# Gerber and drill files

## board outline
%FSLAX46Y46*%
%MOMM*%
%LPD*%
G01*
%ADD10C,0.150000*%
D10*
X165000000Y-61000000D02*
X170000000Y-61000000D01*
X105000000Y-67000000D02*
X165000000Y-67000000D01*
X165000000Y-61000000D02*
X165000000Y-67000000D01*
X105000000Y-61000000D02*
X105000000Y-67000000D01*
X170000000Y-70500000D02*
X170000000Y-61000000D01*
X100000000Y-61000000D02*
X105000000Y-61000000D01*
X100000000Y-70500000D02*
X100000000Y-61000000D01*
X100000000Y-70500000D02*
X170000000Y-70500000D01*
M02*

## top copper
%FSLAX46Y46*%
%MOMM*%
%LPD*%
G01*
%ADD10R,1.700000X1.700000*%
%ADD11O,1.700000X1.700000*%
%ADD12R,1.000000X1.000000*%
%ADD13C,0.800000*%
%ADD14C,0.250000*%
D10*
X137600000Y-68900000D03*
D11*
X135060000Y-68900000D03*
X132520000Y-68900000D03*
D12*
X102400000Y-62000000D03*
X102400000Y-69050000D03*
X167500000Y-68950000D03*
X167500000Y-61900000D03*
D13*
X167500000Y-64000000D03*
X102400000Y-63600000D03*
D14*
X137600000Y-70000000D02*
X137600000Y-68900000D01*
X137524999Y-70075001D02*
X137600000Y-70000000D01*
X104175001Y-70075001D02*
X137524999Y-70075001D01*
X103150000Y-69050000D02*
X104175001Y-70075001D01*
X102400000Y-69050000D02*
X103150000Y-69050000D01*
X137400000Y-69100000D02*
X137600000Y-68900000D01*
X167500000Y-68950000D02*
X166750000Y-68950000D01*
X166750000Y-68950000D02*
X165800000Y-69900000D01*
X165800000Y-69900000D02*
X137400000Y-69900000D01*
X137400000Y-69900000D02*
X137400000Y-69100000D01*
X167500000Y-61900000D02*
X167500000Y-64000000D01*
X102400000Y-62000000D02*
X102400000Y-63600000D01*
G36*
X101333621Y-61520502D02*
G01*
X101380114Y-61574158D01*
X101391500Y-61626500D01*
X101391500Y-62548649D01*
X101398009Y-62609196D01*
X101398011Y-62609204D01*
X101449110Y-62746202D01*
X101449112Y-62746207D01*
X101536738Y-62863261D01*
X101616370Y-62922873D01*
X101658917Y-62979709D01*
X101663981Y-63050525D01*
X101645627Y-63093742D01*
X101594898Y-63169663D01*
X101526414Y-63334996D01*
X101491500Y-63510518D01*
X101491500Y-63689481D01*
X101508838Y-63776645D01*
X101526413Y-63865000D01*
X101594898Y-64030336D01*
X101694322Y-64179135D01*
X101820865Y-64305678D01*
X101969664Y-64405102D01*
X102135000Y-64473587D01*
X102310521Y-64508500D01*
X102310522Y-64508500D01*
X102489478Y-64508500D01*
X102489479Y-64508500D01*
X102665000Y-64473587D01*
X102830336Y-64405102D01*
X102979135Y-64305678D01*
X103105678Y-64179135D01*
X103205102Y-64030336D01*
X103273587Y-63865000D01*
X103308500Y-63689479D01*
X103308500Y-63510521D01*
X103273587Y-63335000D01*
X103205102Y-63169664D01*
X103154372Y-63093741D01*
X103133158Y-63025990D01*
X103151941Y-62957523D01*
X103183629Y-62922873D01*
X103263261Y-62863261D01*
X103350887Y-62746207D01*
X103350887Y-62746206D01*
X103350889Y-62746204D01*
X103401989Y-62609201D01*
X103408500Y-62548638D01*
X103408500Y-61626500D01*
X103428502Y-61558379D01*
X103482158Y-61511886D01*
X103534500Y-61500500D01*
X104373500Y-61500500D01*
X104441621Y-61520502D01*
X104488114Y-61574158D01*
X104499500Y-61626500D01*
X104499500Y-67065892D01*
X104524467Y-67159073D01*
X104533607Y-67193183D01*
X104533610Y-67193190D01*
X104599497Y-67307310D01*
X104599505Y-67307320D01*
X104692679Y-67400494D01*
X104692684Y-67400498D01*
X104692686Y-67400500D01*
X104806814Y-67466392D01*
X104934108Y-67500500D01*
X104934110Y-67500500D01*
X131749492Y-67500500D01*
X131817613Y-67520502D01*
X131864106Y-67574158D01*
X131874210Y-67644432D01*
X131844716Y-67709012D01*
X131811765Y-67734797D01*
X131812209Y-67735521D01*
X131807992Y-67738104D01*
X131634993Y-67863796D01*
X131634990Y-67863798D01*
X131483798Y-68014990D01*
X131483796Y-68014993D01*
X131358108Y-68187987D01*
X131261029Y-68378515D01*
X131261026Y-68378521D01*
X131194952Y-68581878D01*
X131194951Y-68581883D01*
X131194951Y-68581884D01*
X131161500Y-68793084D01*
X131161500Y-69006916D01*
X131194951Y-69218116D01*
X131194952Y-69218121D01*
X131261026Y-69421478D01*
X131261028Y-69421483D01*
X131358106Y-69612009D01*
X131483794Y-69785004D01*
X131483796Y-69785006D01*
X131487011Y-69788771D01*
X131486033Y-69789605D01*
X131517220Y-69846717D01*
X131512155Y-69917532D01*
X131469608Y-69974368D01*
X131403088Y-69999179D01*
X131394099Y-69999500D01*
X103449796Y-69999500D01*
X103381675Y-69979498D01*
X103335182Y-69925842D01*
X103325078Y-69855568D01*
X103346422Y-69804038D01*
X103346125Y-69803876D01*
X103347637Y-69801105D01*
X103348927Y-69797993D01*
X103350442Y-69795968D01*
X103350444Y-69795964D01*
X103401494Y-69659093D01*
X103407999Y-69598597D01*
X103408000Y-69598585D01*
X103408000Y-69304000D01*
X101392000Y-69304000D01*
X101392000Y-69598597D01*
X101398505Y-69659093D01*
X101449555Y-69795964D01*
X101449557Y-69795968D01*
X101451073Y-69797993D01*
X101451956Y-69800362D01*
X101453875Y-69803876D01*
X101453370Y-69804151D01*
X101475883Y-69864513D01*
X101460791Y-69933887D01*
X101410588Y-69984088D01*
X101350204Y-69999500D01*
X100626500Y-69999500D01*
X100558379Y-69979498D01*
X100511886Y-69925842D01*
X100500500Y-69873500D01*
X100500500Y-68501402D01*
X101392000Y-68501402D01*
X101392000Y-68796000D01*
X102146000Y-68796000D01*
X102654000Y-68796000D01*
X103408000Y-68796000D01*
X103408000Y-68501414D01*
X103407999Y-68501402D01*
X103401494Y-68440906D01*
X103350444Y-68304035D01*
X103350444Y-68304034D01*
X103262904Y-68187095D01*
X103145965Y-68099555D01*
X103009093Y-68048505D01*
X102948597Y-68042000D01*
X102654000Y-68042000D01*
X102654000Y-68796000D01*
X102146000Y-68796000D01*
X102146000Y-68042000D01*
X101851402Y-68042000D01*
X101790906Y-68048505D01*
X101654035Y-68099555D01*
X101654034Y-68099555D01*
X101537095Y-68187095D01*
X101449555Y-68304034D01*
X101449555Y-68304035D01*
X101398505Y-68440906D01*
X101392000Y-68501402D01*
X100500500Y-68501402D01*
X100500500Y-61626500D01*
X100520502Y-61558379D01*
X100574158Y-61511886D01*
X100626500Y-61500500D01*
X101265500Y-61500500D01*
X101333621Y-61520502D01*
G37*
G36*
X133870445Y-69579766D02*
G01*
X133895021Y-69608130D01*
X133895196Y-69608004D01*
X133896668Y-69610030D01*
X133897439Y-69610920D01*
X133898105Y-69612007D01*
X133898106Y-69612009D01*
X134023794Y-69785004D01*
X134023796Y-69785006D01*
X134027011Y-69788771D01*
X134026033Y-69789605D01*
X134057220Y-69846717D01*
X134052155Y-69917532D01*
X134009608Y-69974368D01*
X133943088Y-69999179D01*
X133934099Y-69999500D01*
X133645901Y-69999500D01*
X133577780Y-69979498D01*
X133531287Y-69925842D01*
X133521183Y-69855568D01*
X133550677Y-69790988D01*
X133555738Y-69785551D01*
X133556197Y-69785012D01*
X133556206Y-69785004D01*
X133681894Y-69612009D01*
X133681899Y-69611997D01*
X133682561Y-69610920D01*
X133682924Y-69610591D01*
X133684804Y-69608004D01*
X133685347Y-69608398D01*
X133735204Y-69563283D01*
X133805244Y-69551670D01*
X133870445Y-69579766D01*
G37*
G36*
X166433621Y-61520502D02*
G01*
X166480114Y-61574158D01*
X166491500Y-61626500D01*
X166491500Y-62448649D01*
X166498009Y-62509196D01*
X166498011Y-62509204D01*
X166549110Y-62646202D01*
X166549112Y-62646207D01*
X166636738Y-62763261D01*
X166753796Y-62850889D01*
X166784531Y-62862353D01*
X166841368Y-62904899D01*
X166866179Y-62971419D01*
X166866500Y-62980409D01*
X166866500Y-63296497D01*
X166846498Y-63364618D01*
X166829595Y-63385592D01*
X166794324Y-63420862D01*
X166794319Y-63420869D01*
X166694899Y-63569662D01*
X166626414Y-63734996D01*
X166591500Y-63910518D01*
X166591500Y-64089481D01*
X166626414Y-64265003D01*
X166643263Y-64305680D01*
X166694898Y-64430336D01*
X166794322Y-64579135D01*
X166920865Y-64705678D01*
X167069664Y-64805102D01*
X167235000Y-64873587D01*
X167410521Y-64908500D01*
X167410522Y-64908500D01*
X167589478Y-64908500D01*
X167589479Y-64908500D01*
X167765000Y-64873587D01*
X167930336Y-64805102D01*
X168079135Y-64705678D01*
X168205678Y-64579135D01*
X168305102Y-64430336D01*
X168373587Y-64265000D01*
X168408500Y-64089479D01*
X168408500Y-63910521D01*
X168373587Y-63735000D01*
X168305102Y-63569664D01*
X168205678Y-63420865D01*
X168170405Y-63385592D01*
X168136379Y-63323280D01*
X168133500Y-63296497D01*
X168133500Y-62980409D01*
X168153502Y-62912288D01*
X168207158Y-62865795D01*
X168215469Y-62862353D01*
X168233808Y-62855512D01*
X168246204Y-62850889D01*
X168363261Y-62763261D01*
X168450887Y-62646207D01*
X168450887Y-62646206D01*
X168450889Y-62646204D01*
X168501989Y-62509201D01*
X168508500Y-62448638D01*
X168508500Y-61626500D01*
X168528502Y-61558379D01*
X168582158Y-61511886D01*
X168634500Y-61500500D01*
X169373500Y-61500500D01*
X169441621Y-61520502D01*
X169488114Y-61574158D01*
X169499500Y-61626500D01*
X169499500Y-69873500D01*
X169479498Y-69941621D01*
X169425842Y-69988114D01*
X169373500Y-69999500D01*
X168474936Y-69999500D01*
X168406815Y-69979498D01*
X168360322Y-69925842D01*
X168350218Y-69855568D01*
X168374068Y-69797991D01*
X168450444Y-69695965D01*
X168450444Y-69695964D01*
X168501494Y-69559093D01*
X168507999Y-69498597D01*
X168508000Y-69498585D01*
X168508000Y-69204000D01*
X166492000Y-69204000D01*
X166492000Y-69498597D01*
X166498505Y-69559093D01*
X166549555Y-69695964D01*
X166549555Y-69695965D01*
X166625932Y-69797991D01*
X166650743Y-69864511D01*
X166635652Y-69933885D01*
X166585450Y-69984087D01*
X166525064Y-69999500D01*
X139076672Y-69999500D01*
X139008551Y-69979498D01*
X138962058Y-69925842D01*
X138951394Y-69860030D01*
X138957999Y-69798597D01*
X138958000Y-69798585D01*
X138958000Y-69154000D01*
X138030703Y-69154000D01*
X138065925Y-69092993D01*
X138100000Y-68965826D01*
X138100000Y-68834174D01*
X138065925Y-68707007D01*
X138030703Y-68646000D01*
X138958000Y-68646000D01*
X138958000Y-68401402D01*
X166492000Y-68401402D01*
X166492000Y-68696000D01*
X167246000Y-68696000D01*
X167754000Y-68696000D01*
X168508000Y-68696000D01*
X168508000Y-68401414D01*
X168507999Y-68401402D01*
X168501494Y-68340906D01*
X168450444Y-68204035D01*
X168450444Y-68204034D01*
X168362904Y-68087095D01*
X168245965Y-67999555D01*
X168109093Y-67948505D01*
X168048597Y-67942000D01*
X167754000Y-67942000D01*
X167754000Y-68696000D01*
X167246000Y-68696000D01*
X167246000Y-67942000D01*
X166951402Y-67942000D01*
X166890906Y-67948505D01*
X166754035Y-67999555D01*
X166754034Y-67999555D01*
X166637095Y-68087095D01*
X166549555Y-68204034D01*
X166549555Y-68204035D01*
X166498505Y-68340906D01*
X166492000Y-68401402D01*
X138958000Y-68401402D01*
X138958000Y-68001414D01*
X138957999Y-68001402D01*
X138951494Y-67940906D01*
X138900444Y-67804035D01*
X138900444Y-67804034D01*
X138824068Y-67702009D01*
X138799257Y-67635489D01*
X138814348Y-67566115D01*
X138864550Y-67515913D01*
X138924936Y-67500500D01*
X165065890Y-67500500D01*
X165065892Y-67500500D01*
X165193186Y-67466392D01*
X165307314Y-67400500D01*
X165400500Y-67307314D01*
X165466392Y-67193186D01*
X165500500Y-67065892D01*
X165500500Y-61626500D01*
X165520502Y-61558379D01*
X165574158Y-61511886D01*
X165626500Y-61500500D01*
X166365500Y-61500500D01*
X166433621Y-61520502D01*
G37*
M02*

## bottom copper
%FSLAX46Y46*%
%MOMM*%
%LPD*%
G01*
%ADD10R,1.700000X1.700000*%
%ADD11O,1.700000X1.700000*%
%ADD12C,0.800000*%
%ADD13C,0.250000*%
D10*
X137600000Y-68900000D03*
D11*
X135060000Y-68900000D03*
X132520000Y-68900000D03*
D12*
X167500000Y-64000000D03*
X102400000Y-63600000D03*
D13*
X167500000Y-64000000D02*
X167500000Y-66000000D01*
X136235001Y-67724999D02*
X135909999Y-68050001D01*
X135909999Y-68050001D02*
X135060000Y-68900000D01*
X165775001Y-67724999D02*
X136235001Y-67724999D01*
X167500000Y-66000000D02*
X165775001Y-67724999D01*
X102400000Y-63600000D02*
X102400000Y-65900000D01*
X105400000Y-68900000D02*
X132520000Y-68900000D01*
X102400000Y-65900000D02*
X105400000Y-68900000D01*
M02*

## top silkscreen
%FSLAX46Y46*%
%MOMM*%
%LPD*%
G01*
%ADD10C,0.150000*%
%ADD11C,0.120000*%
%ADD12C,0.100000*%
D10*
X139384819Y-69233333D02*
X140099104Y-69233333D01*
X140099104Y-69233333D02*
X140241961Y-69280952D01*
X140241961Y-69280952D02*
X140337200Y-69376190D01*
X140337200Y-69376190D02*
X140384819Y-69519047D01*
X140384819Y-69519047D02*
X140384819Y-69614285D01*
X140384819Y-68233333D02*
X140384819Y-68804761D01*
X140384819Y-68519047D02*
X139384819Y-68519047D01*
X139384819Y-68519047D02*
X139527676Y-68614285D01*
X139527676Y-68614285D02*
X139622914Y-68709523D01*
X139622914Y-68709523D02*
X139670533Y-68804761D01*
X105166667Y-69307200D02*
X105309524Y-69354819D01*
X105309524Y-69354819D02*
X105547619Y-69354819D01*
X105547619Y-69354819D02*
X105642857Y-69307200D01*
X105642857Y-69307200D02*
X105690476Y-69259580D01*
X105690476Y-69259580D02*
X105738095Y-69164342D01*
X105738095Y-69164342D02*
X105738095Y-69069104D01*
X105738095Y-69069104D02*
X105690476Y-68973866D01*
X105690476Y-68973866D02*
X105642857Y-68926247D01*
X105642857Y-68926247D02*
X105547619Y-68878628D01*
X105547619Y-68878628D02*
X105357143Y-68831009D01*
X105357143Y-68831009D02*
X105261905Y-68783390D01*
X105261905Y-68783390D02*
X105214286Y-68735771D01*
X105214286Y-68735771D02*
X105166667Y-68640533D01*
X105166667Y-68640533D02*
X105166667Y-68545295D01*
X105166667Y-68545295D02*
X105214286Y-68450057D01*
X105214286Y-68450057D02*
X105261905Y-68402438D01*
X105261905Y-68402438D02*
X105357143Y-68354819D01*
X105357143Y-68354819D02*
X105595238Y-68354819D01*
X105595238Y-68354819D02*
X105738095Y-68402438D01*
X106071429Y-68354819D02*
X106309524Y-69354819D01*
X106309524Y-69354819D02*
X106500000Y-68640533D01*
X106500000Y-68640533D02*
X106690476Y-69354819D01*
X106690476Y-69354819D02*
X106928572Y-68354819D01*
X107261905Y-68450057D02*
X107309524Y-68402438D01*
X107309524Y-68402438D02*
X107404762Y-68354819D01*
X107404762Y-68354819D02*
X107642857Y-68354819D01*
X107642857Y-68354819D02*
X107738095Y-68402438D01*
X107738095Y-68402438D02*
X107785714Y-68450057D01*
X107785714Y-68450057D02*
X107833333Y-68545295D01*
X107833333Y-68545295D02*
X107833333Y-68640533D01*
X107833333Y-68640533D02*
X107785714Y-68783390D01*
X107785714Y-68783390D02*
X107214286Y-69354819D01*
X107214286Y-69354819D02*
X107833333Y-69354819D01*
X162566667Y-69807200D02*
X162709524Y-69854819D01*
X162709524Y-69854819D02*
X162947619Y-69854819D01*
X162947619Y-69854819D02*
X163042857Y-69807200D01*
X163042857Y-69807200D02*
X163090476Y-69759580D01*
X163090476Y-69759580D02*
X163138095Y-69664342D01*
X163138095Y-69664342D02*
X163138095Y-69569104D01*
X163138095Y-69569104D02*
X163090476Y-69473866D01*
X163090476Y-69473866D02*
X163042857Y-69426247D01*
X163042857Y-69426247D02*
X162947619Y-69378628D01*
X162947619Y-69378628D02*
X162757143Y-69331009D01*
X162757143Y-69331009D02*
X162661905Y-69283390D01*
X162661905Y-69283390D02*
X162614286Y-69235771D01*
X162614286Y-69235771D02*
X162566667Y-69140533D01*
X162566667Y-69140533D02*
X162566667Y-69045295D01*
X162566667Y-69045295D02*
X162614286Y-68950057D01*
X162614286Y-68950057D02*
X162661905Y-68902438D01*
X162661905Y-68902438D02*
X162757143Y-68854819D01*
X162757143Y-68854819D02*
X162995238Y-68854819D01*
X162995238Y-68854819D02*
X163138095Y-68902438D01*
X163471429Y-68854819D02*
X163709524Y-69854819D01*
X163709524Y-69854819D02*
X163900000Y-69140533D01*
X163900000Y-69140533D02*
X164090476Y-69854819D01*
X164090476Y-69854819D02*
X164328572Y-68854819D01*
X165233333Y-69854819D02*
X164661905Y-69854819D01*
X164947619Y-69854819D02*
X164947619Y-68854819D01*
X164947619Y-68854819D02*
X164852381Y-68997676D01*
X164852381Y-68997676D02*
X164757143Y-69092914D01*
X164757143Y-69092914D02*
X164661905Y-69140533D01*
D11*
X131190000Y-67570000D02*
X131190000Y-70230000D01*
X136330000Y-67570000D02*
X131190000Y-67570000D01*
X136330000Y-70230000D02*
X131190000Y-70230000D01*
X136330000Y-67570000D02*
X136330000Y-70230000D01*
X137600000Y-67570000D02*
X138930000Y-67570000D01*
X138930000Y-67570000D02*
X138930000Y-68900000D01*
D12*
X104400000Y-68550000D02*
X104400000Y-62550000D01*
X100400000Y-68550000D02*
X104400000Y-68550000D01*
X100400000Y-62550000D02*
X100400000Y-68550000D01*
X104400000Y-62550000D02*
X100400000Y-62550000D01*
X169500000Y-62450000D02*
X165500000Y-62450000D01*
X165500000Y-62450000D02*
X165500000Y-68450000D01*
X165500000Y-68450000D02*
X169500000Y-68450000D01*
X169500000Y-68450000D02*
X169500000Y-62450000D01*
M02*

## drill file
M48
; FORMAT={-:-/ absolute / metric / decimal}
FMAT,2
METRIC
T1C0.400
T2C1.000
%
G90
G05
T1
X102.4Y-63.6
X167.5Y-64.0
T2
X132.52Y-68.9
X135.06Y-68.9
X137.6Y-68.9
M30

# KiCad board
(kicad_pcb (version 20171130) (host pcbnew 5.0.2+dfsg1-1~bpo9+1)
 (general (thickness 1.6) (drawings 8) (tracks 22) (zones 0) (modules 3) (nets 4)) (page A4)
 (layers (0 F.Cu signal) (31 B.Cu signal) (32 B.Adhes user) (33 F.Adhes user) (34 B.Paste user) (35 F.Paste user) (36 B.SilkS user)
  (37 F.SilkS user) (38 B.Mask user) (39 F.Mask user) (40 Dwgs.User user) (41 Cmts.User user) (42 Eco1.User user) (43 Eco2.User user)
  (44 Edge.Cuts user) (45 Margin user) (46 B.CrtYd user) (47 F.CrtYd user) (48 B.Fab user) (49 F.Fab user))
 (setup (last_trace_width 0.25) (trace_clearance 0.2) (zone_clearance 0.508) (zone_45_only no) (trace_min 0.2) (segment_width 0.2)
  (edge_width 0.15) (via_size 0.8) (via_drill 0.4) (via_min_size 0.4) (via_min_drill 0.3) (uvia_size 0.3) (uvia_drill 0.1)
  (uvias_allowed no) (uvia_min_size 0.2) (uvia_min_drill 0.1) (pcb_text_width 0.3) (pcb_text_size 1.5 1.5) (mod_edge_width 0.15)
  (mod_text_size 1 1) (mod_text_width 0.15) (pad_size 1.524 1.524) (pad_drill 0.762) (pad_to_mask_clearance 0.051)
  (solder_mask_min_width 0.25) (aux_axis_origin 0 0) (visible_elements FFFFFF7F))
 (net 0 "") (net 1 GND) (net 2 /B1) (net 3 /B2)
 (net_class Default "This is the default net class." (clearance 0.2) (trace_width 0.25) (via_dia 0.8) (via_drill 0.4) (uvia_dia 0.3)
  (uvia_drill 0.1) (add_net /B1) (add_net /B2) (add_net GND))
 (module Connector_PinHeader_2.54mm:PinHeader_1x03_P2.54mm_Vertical (layer F.Cu) (at 137.6 68.9 270)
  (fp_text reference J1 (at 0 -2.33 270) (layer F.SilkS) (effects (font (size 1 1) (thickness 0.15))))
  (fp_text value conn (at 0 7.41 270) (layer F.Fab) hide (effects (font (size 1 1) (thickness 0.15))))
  (fp_line (start -1.33 6.41) (end 1.33 6.41) (layer F.SilkS) (width 0.12))
  (fp_line (start -1.33 1.27) (end -1.33 6.41) (layer F.SilkS) (width 0.12))
  (fp_line (start 1.33 1.27) (end 1.33 6.41) (layer F.SilkS) (width 0.12))
  (fp_line (start -1.33 1.27) (end 1.33 1.27) (layer F.SilkS) (width 0.12))
  (fp_line (start -1.33 0) (end -1.33 -1.33) (layer F.SilkS) (width 0.12))
  (fp_line (start -1.33 -1.33) (end 0 -1.33) (layer F.SilkS) (width 0.12))
  (pad 1 thru_hole rect (at 0 0 270) (size 1.7 1.7) (drill 1) (layers *.Cu *.Mask) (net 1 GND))
  (pad 2 thru_hole oval (at 0 2.54 270) (size 1.7 1.7) (drill 1) (layers *.Cu *.Mask) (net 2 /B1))
  (pad 3 thru_hole oval (at 0 5.08 270) (size 1.7 1.7) (drill 1) (layers *.Cu *.Mask) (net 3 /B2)))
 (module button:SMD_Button (layer F.Cu) (at 102.2 65.7 270)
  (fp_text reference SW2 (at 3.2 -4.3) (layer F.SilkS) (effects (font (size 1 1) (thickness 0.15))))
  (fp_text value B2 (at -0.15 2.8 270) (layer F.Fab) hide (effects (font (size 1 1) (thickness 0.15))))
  (fp_line (start 2.85 -2.2) (end -3.15 -2.2) (layer F.SilkS) (width 0.1))
  (fp_line (start 2.85 1.8) (end 2.85 -2.2) (layer F.SilkS) (width 0.1))
  (fp_line (start -3.15 1.8) (end 2.85 1.8) (layer F.SilkS) (width 0.1))
  (fp_line (start -3.15 -2.2) (end -3.15 1.8) (layer F.SilkS) (width 0.1))
  (pad 2 smd rect (at -3.7 -0.2 270) (size 1 1) (layers F.Cu F.Paste F.Mask) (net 3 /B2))
  (pad 1 smd rect (at 3.35 -0.2 270) (size 1 1) (layers F.Cu F.Paste F.Mask) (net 1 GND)))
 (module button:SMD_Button (layer F.Cu) (at 167.3 65.6 270)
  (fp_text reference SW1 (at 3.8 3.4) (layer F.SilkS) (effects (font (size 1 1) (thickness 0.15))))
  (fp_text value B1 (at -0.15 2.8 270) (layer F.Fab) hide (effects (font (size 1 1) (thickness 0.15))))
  (fp_line (start -3.15 -2.2) (end -3.15 1.8) (layer F.SilkS) (width 0.1))
  (fp_line (start -3.15 1.8) (end 2.85 1.8) (layer F.SilkS) (width 0.1))
  (fp_line (start 2.85 1.8) (end 2.85 -2.2) (layer F.SilkS) (width 0.1))
  (fp_line (start 2.85 -2.2) (end -3.15 -2.2) (layer F.SilkS) (width 0.1))
  (pad 1 smd rect (at 3.35 -0.2 270) (size 1 1) (layers F.Cu F.Paste F.Mask) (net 1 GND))
  (pad 2 smd rect (at -3.7 -0.2 270) (size 1 1) (layers F.Cu F.Paste F.Mask) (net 2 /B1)))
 (gr_line (start 165 61) (end 170 61) (layer Edge.Cuts) (width 0.15))
 (gr_line (start 105 67) (end 165 67) (layer Edge.Cuts) (width 0.15))
 (gr_line (start 165 61) (end 165 67) (layer Edge.Cuts) (width 0.15))
 (gr_line (start 105 61) (end 105 67) (layer Edge.Cuts) (width 0.15))
 (gr_line (start 170 70.5) (end 170 61) (layer Edge.Cuts) (width 0.15))
 (gr_line (start 100 61) (end 105 61) (layer Edge.Cuts) (width 0.15))
 (gr_line (start 100 70.5) (end 100 61) (layer Edge.Cuts) (width 0.15))
 (gr_line (start 100 70.5) (end 170 70.5) (layer Edge.Cuts) (width 0.15))
 (segment (start 137.6 70) (end 137.6 68.9) (width 0.25) (layer F.Cu) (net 1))
 (segment (start 137.524999 70.075001) (end 137.6 70) (width 0.25) (layer F.Cu) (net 1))
 (segment (start 104.175001 70.075001) (end 137.524999 70.075001) (width 0.25) (layer F.Cu) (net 1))
 (segment (start 103.15 69.05) (end 104.175001 70.075001) (width 0.25) (layer F.Cu) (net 1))
 (segment (start 102.4 69.05) (end 103.15 69.05) (width 0.25) (layer F.Cu) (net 1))
 (segment (start 137.4 69.1) (end 137.6 68.9) (width 0.25) (layer F.Cu) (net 1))
 (segment (start 167.5 68.95) (end 166.75 68.95) (width 0.25) (layer F.Cu) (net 1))
 (segment (start 166.75 68.95) (end 165.8 69.9) (width 0.25) (layer F.Cu) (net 1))
 (segment (start 165.8 69.9) (end 137.4 69.9) (width 0.25) (layer F.Cu) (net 1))
 (segment (start 137.4 69.9) (end 137.4 69.1) (width 0.25) (layer F.Cu) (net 1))
 (via (at 167.5 64) (size 0.8) (drill 0.4) (layers F.Cu B.Cu) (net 2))
 (segment (start 167.5 61.9) (end 167.5 64) (width 0.25) (layer F.Cu) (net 2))
 (segment (start 167.5 64) (end 167.5 66) (width 0.25) (layer B.Cu) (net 2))
 (segment (start 136.235001 67.724999) (end 135.909999 68.050001) (width 0.25) (layer B.Cu) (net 2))
 (segment (start 135.909999 68.050001) (end 135.06 68.9) (width 0.25) (layer B.Cu) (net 2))
 (segment (start 165.775001 67.724999) (end 136.235001 67.724999) (width 0.25) (layer B.Cu) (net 2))
 (segment (start 167.5 66) (end 165.775001 67.724999) (width 0.25) (layer B.Cu) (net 2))
 (via (at 102.4 63.6) (size 0.8) (drill 0.4) (layers F.Cu B.Cu) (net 3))
 (segment (start 102.4 62) (end 102.4 63.6) (width 0.25) (layer F.Cu) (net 3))
 (segment (start 102.4 63.6) (end 102.4 65.9) (width 0.25) (layer B.Cu) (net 3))
 (segment (start 105.4 68.9) (end 132.52 68.9) (width 0.25) (layer B.Cu) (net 3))
 (segment (start 102.4 65.9) (end 105.4 68.9) (width 0.25) (layer B.Cu) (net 3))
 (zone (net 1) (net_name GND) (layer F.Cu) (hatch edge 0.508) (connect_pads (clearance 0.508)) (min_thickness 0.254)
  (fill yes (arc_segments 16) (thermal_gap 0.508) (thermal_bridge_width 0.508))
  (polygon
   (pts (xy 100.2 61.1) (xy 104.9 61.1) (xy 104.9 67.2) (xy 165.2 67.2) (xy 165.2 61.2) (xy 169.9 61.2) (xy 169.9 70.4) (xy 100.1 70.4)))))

